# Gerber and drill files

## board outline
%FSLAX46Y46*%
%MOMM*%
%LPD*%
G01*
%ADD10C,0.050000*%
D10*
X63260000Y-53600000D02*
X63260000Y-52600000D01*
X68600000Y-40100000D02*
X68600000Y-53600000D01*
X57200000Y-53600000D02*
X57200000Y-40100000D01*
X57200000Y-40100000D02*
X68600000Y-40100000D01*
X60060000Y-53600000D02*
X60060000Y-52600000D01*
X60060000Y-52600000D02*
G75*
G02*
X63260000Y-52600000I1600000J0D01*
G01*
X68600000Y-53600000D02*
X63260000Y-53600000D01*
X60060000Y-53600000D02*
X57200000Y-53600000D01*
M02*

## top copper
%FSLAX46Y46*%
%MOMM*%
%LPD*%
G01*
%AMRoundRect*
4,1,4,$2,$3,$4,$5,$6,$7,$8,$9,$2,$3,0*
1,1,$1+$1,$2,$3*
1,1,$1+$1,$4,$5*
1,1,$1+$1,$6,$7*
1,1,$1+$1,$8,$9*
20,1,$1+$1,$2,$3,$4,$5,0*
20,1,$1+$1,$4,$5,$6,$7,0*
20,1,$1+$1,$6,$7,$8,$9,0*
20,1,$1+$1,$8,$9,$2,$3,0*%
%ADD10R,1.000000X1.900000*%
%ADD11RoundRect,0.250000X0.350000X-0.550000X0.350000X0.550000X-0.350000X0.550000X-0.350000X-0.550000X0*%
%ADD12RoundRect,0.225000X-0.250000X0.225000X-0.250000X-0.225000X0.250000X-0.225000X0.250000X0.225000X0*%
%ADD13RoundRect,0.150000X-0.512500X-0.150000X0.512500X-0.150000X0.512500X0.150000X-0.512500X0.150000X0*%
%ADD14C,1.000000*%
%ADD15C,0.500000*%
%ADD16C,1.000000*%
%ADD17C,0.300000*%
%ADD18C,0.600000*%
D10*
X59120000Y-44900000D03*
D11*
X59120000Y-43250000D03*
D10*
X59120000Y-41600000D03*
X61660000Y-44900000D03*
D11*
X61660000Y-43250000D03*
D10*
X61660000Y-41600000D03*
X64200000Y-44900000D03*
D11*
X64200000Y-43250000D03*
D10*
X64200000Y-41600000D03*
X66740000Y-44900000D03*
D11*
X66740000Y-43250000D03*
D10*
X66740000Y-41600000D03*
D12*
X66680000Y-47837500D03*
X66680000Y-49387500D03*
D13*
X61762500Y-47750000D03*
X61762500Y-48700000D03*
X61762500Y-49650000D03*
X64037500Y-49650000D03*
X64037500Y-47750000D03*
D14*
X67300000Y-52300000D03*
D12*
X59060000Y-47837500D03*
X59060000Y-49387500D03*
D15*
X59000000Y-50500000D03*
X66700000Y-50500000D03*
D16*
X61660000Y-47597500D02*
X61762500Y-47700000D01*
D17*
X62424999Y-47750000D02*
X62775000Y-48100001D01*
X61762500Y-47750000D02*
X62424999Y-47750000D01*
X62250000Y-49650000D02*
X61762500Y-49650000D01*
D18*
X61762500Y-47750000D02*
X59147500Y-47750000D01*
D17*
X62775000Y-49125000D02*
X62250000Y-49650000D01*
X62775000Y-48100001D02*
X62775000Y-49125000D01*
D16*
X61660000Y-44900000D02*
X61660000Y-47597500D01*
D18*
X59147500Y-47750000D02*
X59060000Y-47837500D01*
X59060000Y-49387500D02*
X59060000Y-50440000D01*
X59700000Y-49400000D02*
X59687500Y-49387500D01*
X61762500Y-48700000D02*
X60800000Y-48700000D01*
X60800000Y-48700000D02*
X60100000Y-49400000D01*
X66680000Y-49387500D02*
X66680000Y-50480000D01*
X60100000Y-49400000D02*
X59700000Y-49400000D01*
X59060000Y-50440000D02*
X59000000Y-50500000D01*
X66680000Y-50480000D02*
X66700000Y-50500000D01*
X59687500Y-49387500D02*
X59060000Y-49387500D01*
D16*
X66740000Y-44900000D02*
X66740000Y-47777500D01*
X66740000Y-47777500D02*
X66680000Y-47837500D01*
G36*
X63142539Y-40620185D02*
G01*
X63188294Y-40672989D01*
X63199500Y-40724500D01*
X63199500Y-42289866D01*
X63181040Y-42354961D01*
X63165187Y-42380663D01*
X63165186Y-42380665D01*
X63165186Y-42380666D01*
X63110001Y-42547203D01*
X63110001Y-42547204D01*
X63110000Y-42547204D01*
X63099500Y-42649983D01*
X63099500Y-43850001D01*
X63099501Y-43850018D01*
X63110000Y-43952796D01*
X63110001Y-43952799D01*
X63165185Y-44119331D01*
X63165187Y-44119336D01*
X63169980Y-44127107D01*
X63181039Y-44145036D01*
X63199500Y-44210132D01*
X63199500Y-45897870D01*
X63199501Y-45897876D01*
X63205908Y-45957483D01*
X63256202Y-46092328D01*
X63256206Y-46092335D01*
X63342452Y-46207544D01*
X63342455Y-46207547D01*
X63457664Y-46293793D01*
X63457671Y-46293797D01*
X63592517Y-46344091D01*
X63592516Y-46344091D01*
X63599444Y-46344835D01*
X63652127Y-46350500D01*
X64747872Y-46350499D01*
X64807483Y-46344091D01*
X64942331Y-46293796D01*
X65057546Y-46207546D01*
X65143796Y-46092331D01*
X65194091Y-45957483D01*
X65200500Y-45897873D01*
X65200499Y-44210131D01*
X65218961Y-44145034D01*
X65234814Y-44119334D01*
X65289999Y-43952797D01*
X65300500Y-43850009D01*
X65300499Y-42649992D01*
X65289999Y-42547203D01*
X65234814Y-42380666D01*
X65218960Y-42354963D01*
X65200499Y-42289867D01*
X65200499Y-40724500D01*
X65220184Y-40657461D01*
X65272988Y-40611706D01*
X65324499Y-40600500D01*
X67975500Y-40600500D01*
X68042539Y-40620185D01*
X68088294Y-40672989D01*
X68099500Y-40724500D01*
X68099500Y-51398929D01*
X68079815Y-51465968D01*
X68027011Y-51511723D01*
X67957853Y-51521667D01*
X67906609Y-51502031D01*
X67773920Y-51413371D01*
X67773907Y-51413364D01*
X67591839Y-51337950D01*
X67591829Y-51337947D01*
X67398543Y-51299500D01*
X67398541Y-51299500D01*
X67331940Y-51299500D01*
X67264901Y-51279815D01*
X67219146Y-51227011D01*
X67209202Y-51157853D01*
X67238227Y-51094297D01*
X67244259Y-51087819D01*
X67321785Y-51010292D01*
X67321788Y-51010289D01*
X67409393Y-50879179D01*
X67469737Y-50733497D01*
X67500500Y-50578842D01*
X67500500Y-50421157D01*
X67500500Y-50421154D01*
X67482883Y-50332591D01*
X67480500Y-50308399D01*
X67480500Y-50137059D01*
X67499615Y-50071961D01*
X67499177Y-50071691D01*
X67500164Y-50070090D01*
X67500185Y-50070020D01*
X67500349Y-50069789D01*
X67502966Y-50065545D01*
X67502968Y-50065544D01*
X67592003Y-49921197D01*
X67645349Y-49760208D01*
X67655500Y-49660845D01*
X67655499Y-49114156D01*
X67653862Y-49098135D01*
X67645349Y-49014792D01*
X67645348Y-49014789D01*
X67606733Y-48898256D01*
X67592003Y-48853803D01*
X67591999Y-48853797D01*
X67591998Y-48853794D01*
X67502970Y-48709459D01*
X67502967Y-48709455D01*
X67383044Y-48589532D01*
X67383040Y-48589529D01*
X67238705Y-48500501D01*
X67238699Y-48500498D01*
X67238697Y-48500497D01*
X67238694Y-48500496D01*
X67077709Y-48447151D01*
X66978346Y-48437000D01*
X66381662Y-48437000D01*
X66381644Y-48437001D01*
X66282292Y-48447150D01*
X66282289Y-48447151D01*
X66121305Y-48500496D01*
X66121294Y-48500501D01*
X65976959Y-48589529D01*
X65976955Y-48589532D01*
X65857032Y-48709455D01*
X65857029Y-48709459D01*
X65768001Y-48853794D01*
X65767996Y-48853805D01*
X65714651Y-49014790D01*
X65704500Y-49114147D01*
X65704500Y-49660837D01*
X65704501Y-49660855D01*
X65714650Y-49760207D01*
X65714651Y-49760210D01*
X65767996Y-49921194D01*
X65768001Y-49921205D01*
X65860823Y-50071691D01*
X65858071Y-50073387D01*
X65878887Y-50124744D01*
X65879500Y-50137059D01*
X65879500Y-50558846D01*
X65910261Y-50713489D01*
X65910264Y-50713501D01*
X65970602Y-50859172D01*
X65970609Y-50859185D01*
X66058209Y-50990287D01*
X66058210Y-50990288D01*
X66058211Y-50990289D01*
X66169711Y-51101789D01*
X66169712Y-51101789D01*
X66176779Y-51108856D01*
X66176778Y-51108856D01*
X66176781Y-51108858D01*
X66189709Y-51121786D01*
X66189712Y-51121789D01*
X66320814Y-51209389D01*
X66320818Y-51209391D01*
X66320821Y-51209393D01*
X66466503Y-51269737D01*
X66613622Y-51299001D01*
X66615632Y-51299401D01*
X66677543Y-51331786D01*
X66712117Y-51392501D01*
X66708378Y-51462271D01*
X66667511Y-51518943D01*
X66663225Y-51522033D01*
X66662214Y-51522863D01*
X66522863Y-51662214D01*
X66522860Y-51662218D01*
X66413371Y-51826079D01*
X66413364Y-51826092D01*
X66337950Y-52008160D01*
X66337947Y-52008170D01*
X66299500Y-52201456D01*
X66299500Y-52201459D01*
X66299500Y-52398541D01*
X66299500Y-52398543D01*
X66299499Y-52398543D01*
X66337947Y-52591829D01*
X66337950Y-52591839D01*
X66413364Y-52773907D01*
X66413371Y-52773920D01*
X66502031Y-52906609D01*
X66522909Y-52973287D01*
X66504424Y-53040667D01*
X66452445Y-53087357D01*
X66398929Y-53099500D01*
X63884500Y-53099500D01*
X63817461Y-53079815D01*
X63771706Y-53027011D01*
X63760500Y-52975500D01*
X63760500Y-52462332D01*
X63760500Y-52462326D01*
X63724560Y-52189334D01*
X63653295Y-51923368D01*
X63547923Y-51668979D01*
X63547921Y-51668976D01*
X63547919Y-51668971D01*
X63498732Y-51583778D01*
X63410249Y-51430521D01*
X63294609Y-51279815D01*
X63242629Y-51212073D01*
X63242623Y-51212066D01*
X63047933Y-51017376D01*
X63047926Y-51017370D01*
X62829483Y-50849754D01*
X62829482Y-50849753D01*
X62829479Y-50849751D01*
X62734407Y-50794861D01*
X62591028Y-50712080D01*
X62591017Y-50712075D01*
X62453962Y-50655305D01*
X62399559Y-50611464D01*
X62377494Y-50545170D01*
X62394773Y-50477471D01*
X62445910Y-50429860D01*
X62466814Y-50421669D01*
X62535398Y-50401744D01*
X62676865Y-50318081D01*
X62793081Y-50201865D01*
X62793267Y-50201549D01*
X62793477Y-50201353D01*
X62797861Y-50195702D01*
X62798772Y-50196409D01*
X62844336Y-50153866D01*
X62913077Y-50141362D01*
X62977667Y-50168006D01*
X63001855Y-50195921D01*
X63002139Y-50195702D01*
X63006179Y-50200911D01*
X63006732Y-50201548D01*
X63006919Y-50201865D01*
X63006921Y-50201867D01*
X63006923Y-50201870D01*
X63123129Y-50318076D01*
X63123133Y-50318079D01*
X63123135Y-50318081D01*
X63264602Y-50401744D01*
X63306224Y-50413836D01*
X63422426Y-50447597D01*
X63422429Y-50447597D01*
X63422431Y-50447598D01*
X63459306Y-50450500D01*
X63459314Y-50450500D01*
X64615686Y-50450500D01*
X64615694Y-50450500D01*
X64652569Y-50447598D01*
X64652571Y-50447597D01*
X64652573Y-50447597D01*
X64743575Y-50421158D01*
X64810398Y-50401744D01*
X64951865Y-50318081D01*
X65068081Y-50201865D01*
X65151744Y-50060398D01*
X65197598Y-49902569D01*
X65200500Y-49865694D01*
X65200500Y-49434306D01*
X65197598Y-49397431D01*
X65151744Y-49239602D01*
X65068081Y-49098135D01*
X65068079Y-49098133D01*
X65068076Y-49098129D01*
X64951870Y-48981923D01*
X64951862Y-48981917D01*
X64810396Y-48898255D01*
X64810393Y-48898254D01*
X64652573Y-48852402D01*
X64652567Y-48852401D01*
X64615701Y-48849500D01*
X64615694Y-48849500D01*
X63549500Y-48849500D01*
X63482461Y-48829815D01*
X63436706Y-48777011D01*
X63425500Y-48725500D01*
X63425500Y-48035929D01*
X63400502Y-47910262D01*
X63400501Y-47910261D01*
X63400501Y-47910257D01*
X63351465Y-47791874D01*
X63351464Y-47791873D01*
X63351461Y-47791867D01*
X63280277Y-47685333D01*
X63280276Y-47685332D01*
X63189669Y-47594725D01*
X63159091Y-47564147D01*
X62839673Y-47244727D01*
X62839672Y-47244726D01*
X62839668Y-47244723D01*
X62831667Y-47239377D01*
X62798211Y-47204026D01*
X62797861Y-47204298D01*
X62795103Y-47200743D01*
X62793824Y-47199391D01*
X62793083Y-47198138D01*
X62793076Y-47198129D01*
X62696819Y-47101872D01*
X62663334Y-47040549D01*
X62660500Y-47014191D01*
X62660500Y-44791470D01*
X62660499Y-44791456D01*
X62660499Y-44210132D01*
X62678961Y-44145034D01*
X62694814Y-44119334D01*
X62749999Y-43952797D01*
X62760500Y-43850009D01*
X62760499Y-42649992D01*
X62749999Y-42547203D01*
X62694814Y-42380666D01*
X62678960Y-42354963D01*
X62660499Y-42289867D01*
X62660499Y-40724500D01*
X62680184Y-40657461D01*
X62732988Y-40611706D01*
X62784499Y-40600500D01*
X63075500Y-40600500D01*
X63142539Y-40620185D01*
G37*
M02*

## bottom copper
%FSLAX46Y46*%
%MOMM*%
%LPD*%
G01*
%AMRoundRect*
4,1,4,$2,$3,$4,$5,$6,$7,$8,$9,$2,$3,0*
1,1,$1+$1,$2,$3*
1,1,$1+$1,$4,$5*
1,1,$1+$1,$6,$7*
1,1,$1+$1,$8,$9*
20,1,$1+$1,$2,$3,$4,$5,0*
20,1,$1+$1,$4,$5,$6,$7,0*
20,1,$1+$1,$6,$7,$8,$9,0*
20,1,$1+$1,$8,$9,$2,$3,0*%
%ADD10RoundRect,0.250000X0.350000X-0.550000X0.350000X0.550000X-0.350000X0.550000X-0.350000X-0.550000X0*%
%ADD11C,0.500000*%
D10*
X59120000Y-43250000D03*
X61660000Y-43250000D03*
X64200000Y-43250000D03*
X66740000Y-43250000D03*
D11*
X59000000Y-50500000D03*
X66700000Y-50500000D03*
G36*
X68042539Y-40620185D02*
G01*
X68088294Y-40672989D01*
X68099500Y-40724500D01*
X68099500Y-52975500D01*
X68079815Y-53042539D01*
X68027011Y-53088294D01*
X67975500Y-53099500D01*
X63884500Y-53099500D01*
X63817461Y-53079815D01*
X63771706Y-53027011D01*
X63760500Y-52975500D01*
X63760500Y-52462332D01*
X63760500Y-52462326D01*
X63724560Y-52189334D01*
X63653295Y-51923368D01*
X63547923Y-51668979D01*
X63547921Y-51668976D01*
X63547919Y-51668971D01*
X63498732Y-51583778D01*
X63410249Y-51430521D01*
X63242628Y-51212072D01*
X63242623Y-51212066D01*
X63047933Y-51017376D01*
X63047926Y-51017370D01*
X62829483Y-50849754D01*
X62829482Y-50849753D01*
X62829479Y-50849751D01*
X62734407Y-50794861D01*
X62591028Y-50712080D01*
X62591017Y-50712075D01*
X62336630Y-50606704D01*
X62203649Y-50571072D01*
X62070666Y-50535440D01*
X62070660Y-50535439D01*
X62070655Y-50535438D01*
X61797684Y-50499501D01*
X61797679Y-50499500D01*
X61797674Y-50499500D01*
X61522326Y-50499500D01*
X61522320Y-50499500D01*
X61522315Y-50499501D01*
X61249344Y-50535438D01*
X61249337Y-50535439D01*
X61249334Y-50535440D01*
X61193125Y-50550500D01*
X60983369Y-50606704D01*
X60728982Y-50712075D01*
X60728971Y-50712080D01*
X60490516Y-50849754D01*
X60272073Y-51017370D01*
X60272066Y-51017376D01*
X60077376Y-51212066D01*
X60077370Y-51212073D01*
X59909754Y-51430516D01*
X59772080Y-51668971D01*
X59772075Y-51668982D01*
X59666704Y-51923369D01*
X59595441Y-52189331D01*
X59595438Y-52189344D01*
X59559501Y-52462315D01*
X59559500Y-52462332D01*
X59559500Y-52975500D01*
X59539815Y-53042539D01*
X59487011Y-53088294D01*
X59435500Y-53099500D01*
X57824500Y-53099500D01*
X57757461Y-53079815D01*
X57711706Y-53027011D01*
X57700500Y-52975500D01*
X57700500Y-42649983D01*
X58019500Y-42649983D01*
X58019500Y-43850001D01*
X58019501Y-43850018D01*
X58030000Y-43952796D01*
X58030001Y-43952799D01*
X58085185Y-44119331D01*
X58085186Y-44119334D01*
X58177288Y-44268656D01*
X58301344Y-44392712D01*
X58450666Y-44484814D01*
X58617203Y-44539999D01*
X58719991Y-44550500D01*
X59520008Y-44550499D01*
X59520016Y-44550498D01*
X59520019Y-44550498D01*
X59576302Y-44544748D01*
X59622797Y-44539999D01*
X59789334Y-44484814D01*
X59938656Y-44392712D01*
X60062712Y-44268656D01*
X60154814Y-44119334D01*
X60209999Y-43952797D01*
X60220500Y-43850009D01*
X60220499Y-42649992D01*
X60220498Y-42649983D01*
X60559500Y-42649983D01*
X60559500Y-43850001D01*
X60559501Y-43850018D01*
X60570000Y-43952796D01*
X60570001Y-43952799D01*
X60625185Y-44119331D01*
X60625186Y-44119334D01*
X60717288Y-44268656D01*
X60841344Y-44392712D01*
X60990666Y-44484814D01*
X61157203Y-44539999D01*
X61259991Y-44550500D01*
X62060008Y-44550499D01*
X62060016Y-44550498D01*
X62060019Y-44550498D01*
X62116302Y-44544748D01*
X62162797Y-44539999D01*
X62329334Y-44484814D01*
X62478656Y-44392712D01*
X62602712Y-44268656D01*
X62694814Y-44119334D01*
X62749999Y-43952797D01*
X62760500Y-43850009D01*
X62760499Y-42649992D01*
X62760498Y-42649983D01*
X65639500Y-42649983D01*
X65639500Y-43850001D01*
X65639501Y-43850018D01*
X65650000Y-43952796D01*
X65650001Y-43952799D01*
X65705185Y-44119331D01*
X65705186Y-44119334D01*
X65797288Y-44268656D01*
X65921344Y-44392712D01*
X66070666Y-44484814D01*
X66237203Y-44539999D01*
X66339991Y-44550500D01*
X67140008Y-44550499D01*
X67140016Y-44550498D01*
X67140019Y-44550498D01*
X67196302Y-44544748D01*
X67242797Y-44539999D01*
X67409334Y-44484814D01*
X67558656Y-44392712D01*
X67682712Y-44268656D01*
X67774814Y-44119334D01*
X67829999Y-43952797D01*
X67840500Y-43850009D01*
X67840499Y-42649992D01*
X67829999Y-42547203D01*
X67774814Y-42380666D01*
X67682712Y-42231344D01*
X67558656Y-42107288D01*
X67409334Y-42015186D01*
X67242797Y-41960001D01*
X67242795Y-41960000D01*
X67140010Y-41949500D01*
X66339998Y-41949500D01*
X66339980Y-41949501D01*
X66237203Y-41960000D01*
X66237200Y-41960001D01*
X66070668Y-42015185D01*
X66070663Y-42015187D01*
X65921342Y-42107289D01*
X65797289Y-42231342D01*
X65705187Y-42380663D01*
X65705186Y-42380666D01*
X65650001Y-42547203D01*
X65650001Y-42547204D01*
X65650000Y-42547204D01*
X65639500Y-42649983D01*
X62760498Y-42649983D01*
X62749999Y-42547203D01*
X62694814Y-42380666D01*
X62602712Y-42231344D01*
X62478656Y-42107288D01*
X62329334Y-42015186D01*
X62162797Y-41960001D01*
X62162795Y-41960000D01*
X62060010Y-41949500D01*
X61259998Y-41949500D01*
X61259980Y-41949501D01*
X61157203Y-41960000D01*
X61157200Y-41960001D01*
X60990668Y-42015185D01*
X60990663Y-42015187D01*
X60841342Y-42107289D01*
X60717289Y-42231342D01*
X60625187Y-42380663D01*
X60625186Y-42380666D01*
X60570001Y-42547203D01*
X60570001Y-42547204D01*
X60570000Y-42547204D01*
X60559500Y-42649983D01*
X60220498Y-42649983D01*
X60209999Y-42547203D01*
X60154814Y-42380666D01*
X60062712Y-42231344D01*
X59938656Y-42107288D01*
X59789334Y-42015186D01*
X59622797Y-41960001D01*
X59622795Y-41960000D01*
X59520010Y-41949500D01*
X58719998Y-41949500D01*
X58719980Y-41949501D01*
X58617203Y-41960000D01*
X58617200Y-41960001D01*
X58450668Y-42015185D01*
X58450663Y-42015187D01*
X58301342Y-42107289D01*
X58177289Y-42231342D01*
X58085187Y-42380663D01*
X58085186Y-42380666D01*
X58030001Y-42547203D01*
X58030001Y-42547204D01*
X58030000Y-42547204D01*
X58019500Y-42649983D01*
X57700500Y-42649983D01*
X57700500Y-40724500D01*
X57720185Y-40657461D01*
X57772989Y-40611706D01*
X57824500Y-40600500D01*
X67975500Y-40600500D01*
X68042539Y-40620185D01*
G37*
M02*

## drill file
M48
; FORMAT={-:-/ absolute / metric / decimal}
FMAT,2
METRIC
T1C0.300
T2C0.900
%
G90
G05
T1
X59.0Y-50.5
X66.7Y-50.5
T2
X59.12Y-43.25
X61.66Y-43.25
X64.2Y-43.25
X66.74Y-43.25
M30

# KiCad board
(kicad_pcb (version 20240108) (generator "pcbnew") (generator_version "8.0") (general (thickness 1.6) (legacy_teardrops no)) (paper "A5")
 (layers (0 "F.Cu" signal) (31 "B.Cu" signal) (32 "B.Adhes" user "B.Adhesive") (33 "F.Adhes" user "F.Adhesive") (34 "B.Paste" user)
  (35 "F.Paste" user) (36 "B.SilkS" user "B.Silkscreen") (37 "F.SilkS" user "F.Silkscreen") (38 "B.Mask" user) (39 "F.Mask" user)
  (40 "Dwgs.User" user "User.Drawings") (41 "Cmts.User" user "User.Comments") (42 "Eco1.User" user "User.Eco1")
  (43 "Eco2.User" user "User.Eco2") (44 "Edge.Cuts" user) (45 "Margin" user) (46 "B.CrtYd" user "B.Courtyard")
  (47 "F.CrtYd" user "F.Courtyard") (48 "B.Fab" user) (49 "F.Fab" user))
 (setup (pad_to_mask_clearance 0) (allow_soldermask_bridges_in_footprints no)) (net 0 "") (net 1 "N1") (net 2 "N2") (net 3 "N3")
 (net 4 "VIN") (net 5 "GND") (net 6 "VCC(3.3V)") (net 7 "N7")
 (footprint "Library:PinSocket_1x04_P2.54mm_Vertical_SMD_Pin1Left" (layer "F.Cu") (at 62.93 43.25 90)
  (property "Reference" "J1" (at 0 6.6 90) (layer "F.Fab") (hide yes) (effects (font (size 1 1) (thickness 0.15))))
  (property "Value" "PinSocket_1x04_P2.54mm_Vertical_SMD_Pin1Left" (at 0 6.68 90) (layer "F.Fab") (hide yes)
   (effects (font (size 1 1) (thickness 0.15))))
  (pad "1" smd rect (at -1.65 -3.81 90) (size 1.9 1) (layers "F.Cu" "F.Paste" "F.Mask") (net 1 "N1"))
  (pad "1" thru_hole roundrect (at 0 -3.81 90) (size 1.6 1.2) (drill 0.9) (layers "*.Cu" "*.Mask") (remove_unused_layers no)
   (roundrect_rratio 0.2083333333) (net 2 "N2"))
  (pad "1" smd rect (at 1.65 -3.81 90) (size 1.9 1) (layers "F.Cu" "F.Paste" "F.Mask") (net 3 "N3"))
  (pad "2" smd rect (at -1.65 -1.27 90) (size 1.9 1) (layers "F.Cu" "F.Paste" "F.Mask") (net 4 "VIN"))
  (pad "2" thru_hole roundrect (at 0 -1.27 90) (size 1.6 1.2) (drill 0.9) (layers "*.Cu" "*.Mask") (remove_unused_layers no)
   (roundrect_rratio 0.2083333333) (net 4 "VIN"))
  (pad "2" smd rect (at 1.65 -1.27 90) (size 1.9 1) (layers "F.Cu" "F.Paste" "F.Mask") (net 4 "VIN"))
  (pad "3" smd rect (at -1.65 1.27 90) (size 1.9 1) (layers "F.Cu" "F.Paste" "F.Mask") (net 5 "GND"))
  (pad "3" thru_hole roundrect (at 0 1.27 90) (size 1.6 1.2) (drill 0.9) (layers "*.Cu" "*.Mask") (remove_unused_layers no)
   (roundrect_rratio 0.2083333333) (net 5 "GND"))
  (pad "3" smd rect (at 1.65 1.27 90) (size 1.9 1) (layers "F.Cu" "F.Paste" "F.Mask") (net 5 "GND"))
  (pad "4" smd rect (at -1.65 3.81 90) (size 1.9 1) (layers "F.Cu" "F.Paste" "F.Mask") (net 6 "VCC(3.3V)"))
  (pad "4" thru_hole roundrect (at 0 3.81 90) (size 1.6 1.2) (drill 0.9) (layers "*.Cu" "*.Mask") (remove_unused_layers no)
   (roundrect_rratio 0.2083333333) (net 6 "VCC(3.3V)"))
  (pad "4" smd rect (at 1.65 3.81 90) (size 1.9 1) (layers "F.Cu" "F.Paste" "F.Mask") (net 6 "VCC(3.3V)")))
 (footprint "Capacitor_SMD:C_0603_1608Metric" (layer "F.Cu") (at 66.68 48.6125 -90)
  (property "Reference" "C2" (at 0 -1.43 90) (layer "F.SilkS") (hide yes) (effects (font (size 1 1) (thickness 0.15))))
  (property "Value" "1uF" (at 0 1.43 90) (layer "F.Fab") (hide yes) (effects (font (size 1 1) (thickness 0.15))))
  (pad "1" smd roundrect (at -0.775 0 270) (size 0.9 0.95) (layers "F.Cu" "F.Paste" "F.Mask") (roundrect_rratio 0.25) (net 6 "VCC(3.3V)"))
  (pad "2" smd roundrect (at 0.775 0 270) (size 0.9 0.95) (layers "F.Cu" "F.Paste" "F.Mask") (roundrect_rratio 0.25) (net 5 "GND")))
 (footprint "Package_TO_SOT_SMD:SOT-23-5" (layer "F.Cu") (at 62.9 48.7)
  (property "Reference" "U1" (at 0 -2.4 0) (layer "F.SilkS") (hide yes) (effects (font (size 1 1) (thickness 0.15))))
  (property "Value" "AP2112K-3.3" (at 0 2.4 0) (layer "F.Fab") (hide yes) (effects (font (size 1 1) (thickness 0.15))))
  (pad "1" smd roundrect (at -1.1375 -0.95) (size 1.325 0.6) (layers "F.Cu" "F.Paste" "F.Mask") (roundrect_rratio 0.25) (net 4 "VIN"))
  (pad "2" smd roundrect (at -1.1375 0) (size 1.325 0.6) (layers "F.Cu" "F.Paste" "F.Mask") (roundrect_rratio 0.25) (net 5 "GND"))
  (pad "3" smd roundrect (at -1.1375 0.95) (size 1.325 0.6) (layers "F.Cu" "F.Paste" "F.Mask") (roundrect_rratio 0.25) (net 4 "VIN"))
  (pad "4" smd roundrect (at 1.1375 0.95) (size 1.325 0.6) (layers "F.Cu" "F.Paste" "F.Mask") (roundrect_rratio 0.25) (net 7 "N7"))
  (pad "5" smd roundrect (at 1.1375 -0.95) (size 1.325 0.6) (layers "F.Cu" "F.Paste" "F.Mask") (roundrect_rratio 0.25) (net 6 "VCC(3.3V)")))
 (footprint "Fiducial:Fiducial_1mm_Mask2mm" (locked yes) (layer "F.Cu") (at 67.3 52.3)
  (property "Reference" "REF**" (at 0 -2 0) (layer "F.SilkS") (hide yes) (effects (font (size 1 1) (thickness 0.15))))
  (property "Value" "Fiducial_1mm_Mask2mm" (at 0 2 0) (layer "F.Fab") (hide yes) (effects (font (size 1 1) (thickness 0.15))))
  (pad "" smd circle (at 0 0) (size 1 1) (layers "F.Cu" "F.Mask") (solder_mask_margin 0.5) (clearance 0.5)))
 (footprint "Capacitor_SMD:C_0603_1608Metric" (layer "F.Cu") (at 59.06 48.6125 -90)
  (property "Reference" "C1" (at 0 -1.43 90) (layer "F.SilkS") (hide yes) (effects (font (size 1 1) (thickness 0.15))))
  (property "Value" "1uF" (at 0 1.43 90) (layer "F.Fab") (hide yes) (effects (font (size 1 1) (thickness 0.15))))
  (pad "1" smd roundrect (at -0.775 0 270) (size 0.9 0.95) (layers "F.Cu" "F.Paste" "F.Mask") (roundrect_rratio 0.25) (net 4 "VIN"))
  (pad "2" smd roundrect (at 0.775 0 270) (size 0.9 0.95) (layers "F.Cu" "F.Paste" "F.Mask") (roundrect_rratio 0.25) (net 5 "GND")))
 (gr_line (start 63.26 53.6) (end 63.26 52.6) (stroke (width 0.05) (type default)) (layer "Edge.Cuts"))
 (gr_line (start 68.6 40.1) (end 68.6 53.6) (stroke (width 0.05) (type default)) (layer "Edge.Cuts"))
 (gr_line (start 57.2 53.6) (end 57.2 40.1) (stroke (width 0.05) (type default)) (layer "Edge.Cuts"))
 (gr_line (start 57.2 40.1) (end 68.6 40.1) (stroke (width 0.05) (type default)) (layer "Edge.Cuts"))
 (gr_line (start 60.06 53.6) (end 60.06 52.6) (stroke (width 0.05) (type default)) (layer "Edge.Cuts"))
 (gr_arc (start 60.06 52.6) (mid 61.66 51) (end 63.26 52.6) (stroke (width 0.05) (type default)) (layer "Edge.Cuts"))
 (gr_line (start 68.6 53.6) (end 63.26 53.6) (stroke (width 0.05) (type default)) (layer "Edge.Cuts"))
 (gr_line (start 60.06 53.6) (end 57.2 53.6) (stroke (width 0.05) (type default)) (layer "Edge.Cuts"))
 (segment (start 61.66 47.5975) (end 61.7625 47.7) (width 1) (layer "F.Cu") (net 4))
 (segment (start 62.424999 47.75) (end 62.775 48.100001) (width 0.3) (layer "F.Cu") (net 4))
 (segment (start 61.7625 47.75) (end 62.424999 47.75) (width 0.3) (layer "F.Cu") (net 4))
 (segment (start 62.25 49.65) (end 61.7625 49.65) (width 0.3) (layer "F.Cu") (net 4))
 (segment (start 61.7625 47.75) (end 59.1475 47.75) (width 0.6) (layer "F.Cu") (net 4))
 (segment (start 62.775 49.125) (end 62.25 49.65) (width 0.3) (layer "F.Cu") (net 4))
 (segment (start 62.775 48.100001) (end 62.775 49.125) (width 0.3) (layer "F.Cu") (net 4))
 (segment (start 61.66 44.9) (end 61.66 47.5975) (width 1) (layer "F.Cu") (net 4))
 (segment (start 59.1475 47.75) (end 59.06 47.8375) (width 0.6) (layer "F.Cu") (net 4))
 (segment (start 59.06 49.3875) (end 59.06 50.44) (width 0.6) (layer "F.Cu") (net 5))
 (segment (start 59.7 49.4) (end 59.6875 49.3875) (width 0.6) (layer "F.Cu") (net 5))
 (segment (start 61.7625 48.7) (end 60.8 48.7) (width 0.6) (layer "F.Cu") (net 5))
 (segment (start 60.8 48.7) (end 60.1 49.4) (width 0.6) (layer "F.Cu") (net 5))
 (segment (start 66.68 49.3875) (end 66.68 50.48) (width 0.6) (layer "F.Cu") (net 5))
 (segment (start 60.1 49.4) (end 59.7 49.4) (width 0.6) (layer "F.Cu") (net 5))
 (segment (start 59.06 50.44) (end 59 50.5) (width 0.6) (layer "F.Cu") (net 5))
 (segment (start 66.68 50.48) (end 66.7 50.5) (width 0.6) (layer "F.Cu") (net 5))
 (segment (start 59.6875 49.3875) (end 59.06 49.3875) (width 0.6) (layer "F.Cu") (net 5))
 (via (at 59 50.5) (size 0.5) (drill 0.3) (layers "F.Cu" "B.Cu") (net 5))
 (via (at 66.7 50.5) (size 0.5) (drill 0.3) (layers "F.Cu" "B.Cu") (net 5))
 (segment (start 66.74 44.9) (end 66.74 47.7775) (width 1) (layer "F.Cu") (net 6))
 (segment (start 66.74 47.7775) (end 66.68 47.8375) (width 1) (layer "F.Cu") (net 6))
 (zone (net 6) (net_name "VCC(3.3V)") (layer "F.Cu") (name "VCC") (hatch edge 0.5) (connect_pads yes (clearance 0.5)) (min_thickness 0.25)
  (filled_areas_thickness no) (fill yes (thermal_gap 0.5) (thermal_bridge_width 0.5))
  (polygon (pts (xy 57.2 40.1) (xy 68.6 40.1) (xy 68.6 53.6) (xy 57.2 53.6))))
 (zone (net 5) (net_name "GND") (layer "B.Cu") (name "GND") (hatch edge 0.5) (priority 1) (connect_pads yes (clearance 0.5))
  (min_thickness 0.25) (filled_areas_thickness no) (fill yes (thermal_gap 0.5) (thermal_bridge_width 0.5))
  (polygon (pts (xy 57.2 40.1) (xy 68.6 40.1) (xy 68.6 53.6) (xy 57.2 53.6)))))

